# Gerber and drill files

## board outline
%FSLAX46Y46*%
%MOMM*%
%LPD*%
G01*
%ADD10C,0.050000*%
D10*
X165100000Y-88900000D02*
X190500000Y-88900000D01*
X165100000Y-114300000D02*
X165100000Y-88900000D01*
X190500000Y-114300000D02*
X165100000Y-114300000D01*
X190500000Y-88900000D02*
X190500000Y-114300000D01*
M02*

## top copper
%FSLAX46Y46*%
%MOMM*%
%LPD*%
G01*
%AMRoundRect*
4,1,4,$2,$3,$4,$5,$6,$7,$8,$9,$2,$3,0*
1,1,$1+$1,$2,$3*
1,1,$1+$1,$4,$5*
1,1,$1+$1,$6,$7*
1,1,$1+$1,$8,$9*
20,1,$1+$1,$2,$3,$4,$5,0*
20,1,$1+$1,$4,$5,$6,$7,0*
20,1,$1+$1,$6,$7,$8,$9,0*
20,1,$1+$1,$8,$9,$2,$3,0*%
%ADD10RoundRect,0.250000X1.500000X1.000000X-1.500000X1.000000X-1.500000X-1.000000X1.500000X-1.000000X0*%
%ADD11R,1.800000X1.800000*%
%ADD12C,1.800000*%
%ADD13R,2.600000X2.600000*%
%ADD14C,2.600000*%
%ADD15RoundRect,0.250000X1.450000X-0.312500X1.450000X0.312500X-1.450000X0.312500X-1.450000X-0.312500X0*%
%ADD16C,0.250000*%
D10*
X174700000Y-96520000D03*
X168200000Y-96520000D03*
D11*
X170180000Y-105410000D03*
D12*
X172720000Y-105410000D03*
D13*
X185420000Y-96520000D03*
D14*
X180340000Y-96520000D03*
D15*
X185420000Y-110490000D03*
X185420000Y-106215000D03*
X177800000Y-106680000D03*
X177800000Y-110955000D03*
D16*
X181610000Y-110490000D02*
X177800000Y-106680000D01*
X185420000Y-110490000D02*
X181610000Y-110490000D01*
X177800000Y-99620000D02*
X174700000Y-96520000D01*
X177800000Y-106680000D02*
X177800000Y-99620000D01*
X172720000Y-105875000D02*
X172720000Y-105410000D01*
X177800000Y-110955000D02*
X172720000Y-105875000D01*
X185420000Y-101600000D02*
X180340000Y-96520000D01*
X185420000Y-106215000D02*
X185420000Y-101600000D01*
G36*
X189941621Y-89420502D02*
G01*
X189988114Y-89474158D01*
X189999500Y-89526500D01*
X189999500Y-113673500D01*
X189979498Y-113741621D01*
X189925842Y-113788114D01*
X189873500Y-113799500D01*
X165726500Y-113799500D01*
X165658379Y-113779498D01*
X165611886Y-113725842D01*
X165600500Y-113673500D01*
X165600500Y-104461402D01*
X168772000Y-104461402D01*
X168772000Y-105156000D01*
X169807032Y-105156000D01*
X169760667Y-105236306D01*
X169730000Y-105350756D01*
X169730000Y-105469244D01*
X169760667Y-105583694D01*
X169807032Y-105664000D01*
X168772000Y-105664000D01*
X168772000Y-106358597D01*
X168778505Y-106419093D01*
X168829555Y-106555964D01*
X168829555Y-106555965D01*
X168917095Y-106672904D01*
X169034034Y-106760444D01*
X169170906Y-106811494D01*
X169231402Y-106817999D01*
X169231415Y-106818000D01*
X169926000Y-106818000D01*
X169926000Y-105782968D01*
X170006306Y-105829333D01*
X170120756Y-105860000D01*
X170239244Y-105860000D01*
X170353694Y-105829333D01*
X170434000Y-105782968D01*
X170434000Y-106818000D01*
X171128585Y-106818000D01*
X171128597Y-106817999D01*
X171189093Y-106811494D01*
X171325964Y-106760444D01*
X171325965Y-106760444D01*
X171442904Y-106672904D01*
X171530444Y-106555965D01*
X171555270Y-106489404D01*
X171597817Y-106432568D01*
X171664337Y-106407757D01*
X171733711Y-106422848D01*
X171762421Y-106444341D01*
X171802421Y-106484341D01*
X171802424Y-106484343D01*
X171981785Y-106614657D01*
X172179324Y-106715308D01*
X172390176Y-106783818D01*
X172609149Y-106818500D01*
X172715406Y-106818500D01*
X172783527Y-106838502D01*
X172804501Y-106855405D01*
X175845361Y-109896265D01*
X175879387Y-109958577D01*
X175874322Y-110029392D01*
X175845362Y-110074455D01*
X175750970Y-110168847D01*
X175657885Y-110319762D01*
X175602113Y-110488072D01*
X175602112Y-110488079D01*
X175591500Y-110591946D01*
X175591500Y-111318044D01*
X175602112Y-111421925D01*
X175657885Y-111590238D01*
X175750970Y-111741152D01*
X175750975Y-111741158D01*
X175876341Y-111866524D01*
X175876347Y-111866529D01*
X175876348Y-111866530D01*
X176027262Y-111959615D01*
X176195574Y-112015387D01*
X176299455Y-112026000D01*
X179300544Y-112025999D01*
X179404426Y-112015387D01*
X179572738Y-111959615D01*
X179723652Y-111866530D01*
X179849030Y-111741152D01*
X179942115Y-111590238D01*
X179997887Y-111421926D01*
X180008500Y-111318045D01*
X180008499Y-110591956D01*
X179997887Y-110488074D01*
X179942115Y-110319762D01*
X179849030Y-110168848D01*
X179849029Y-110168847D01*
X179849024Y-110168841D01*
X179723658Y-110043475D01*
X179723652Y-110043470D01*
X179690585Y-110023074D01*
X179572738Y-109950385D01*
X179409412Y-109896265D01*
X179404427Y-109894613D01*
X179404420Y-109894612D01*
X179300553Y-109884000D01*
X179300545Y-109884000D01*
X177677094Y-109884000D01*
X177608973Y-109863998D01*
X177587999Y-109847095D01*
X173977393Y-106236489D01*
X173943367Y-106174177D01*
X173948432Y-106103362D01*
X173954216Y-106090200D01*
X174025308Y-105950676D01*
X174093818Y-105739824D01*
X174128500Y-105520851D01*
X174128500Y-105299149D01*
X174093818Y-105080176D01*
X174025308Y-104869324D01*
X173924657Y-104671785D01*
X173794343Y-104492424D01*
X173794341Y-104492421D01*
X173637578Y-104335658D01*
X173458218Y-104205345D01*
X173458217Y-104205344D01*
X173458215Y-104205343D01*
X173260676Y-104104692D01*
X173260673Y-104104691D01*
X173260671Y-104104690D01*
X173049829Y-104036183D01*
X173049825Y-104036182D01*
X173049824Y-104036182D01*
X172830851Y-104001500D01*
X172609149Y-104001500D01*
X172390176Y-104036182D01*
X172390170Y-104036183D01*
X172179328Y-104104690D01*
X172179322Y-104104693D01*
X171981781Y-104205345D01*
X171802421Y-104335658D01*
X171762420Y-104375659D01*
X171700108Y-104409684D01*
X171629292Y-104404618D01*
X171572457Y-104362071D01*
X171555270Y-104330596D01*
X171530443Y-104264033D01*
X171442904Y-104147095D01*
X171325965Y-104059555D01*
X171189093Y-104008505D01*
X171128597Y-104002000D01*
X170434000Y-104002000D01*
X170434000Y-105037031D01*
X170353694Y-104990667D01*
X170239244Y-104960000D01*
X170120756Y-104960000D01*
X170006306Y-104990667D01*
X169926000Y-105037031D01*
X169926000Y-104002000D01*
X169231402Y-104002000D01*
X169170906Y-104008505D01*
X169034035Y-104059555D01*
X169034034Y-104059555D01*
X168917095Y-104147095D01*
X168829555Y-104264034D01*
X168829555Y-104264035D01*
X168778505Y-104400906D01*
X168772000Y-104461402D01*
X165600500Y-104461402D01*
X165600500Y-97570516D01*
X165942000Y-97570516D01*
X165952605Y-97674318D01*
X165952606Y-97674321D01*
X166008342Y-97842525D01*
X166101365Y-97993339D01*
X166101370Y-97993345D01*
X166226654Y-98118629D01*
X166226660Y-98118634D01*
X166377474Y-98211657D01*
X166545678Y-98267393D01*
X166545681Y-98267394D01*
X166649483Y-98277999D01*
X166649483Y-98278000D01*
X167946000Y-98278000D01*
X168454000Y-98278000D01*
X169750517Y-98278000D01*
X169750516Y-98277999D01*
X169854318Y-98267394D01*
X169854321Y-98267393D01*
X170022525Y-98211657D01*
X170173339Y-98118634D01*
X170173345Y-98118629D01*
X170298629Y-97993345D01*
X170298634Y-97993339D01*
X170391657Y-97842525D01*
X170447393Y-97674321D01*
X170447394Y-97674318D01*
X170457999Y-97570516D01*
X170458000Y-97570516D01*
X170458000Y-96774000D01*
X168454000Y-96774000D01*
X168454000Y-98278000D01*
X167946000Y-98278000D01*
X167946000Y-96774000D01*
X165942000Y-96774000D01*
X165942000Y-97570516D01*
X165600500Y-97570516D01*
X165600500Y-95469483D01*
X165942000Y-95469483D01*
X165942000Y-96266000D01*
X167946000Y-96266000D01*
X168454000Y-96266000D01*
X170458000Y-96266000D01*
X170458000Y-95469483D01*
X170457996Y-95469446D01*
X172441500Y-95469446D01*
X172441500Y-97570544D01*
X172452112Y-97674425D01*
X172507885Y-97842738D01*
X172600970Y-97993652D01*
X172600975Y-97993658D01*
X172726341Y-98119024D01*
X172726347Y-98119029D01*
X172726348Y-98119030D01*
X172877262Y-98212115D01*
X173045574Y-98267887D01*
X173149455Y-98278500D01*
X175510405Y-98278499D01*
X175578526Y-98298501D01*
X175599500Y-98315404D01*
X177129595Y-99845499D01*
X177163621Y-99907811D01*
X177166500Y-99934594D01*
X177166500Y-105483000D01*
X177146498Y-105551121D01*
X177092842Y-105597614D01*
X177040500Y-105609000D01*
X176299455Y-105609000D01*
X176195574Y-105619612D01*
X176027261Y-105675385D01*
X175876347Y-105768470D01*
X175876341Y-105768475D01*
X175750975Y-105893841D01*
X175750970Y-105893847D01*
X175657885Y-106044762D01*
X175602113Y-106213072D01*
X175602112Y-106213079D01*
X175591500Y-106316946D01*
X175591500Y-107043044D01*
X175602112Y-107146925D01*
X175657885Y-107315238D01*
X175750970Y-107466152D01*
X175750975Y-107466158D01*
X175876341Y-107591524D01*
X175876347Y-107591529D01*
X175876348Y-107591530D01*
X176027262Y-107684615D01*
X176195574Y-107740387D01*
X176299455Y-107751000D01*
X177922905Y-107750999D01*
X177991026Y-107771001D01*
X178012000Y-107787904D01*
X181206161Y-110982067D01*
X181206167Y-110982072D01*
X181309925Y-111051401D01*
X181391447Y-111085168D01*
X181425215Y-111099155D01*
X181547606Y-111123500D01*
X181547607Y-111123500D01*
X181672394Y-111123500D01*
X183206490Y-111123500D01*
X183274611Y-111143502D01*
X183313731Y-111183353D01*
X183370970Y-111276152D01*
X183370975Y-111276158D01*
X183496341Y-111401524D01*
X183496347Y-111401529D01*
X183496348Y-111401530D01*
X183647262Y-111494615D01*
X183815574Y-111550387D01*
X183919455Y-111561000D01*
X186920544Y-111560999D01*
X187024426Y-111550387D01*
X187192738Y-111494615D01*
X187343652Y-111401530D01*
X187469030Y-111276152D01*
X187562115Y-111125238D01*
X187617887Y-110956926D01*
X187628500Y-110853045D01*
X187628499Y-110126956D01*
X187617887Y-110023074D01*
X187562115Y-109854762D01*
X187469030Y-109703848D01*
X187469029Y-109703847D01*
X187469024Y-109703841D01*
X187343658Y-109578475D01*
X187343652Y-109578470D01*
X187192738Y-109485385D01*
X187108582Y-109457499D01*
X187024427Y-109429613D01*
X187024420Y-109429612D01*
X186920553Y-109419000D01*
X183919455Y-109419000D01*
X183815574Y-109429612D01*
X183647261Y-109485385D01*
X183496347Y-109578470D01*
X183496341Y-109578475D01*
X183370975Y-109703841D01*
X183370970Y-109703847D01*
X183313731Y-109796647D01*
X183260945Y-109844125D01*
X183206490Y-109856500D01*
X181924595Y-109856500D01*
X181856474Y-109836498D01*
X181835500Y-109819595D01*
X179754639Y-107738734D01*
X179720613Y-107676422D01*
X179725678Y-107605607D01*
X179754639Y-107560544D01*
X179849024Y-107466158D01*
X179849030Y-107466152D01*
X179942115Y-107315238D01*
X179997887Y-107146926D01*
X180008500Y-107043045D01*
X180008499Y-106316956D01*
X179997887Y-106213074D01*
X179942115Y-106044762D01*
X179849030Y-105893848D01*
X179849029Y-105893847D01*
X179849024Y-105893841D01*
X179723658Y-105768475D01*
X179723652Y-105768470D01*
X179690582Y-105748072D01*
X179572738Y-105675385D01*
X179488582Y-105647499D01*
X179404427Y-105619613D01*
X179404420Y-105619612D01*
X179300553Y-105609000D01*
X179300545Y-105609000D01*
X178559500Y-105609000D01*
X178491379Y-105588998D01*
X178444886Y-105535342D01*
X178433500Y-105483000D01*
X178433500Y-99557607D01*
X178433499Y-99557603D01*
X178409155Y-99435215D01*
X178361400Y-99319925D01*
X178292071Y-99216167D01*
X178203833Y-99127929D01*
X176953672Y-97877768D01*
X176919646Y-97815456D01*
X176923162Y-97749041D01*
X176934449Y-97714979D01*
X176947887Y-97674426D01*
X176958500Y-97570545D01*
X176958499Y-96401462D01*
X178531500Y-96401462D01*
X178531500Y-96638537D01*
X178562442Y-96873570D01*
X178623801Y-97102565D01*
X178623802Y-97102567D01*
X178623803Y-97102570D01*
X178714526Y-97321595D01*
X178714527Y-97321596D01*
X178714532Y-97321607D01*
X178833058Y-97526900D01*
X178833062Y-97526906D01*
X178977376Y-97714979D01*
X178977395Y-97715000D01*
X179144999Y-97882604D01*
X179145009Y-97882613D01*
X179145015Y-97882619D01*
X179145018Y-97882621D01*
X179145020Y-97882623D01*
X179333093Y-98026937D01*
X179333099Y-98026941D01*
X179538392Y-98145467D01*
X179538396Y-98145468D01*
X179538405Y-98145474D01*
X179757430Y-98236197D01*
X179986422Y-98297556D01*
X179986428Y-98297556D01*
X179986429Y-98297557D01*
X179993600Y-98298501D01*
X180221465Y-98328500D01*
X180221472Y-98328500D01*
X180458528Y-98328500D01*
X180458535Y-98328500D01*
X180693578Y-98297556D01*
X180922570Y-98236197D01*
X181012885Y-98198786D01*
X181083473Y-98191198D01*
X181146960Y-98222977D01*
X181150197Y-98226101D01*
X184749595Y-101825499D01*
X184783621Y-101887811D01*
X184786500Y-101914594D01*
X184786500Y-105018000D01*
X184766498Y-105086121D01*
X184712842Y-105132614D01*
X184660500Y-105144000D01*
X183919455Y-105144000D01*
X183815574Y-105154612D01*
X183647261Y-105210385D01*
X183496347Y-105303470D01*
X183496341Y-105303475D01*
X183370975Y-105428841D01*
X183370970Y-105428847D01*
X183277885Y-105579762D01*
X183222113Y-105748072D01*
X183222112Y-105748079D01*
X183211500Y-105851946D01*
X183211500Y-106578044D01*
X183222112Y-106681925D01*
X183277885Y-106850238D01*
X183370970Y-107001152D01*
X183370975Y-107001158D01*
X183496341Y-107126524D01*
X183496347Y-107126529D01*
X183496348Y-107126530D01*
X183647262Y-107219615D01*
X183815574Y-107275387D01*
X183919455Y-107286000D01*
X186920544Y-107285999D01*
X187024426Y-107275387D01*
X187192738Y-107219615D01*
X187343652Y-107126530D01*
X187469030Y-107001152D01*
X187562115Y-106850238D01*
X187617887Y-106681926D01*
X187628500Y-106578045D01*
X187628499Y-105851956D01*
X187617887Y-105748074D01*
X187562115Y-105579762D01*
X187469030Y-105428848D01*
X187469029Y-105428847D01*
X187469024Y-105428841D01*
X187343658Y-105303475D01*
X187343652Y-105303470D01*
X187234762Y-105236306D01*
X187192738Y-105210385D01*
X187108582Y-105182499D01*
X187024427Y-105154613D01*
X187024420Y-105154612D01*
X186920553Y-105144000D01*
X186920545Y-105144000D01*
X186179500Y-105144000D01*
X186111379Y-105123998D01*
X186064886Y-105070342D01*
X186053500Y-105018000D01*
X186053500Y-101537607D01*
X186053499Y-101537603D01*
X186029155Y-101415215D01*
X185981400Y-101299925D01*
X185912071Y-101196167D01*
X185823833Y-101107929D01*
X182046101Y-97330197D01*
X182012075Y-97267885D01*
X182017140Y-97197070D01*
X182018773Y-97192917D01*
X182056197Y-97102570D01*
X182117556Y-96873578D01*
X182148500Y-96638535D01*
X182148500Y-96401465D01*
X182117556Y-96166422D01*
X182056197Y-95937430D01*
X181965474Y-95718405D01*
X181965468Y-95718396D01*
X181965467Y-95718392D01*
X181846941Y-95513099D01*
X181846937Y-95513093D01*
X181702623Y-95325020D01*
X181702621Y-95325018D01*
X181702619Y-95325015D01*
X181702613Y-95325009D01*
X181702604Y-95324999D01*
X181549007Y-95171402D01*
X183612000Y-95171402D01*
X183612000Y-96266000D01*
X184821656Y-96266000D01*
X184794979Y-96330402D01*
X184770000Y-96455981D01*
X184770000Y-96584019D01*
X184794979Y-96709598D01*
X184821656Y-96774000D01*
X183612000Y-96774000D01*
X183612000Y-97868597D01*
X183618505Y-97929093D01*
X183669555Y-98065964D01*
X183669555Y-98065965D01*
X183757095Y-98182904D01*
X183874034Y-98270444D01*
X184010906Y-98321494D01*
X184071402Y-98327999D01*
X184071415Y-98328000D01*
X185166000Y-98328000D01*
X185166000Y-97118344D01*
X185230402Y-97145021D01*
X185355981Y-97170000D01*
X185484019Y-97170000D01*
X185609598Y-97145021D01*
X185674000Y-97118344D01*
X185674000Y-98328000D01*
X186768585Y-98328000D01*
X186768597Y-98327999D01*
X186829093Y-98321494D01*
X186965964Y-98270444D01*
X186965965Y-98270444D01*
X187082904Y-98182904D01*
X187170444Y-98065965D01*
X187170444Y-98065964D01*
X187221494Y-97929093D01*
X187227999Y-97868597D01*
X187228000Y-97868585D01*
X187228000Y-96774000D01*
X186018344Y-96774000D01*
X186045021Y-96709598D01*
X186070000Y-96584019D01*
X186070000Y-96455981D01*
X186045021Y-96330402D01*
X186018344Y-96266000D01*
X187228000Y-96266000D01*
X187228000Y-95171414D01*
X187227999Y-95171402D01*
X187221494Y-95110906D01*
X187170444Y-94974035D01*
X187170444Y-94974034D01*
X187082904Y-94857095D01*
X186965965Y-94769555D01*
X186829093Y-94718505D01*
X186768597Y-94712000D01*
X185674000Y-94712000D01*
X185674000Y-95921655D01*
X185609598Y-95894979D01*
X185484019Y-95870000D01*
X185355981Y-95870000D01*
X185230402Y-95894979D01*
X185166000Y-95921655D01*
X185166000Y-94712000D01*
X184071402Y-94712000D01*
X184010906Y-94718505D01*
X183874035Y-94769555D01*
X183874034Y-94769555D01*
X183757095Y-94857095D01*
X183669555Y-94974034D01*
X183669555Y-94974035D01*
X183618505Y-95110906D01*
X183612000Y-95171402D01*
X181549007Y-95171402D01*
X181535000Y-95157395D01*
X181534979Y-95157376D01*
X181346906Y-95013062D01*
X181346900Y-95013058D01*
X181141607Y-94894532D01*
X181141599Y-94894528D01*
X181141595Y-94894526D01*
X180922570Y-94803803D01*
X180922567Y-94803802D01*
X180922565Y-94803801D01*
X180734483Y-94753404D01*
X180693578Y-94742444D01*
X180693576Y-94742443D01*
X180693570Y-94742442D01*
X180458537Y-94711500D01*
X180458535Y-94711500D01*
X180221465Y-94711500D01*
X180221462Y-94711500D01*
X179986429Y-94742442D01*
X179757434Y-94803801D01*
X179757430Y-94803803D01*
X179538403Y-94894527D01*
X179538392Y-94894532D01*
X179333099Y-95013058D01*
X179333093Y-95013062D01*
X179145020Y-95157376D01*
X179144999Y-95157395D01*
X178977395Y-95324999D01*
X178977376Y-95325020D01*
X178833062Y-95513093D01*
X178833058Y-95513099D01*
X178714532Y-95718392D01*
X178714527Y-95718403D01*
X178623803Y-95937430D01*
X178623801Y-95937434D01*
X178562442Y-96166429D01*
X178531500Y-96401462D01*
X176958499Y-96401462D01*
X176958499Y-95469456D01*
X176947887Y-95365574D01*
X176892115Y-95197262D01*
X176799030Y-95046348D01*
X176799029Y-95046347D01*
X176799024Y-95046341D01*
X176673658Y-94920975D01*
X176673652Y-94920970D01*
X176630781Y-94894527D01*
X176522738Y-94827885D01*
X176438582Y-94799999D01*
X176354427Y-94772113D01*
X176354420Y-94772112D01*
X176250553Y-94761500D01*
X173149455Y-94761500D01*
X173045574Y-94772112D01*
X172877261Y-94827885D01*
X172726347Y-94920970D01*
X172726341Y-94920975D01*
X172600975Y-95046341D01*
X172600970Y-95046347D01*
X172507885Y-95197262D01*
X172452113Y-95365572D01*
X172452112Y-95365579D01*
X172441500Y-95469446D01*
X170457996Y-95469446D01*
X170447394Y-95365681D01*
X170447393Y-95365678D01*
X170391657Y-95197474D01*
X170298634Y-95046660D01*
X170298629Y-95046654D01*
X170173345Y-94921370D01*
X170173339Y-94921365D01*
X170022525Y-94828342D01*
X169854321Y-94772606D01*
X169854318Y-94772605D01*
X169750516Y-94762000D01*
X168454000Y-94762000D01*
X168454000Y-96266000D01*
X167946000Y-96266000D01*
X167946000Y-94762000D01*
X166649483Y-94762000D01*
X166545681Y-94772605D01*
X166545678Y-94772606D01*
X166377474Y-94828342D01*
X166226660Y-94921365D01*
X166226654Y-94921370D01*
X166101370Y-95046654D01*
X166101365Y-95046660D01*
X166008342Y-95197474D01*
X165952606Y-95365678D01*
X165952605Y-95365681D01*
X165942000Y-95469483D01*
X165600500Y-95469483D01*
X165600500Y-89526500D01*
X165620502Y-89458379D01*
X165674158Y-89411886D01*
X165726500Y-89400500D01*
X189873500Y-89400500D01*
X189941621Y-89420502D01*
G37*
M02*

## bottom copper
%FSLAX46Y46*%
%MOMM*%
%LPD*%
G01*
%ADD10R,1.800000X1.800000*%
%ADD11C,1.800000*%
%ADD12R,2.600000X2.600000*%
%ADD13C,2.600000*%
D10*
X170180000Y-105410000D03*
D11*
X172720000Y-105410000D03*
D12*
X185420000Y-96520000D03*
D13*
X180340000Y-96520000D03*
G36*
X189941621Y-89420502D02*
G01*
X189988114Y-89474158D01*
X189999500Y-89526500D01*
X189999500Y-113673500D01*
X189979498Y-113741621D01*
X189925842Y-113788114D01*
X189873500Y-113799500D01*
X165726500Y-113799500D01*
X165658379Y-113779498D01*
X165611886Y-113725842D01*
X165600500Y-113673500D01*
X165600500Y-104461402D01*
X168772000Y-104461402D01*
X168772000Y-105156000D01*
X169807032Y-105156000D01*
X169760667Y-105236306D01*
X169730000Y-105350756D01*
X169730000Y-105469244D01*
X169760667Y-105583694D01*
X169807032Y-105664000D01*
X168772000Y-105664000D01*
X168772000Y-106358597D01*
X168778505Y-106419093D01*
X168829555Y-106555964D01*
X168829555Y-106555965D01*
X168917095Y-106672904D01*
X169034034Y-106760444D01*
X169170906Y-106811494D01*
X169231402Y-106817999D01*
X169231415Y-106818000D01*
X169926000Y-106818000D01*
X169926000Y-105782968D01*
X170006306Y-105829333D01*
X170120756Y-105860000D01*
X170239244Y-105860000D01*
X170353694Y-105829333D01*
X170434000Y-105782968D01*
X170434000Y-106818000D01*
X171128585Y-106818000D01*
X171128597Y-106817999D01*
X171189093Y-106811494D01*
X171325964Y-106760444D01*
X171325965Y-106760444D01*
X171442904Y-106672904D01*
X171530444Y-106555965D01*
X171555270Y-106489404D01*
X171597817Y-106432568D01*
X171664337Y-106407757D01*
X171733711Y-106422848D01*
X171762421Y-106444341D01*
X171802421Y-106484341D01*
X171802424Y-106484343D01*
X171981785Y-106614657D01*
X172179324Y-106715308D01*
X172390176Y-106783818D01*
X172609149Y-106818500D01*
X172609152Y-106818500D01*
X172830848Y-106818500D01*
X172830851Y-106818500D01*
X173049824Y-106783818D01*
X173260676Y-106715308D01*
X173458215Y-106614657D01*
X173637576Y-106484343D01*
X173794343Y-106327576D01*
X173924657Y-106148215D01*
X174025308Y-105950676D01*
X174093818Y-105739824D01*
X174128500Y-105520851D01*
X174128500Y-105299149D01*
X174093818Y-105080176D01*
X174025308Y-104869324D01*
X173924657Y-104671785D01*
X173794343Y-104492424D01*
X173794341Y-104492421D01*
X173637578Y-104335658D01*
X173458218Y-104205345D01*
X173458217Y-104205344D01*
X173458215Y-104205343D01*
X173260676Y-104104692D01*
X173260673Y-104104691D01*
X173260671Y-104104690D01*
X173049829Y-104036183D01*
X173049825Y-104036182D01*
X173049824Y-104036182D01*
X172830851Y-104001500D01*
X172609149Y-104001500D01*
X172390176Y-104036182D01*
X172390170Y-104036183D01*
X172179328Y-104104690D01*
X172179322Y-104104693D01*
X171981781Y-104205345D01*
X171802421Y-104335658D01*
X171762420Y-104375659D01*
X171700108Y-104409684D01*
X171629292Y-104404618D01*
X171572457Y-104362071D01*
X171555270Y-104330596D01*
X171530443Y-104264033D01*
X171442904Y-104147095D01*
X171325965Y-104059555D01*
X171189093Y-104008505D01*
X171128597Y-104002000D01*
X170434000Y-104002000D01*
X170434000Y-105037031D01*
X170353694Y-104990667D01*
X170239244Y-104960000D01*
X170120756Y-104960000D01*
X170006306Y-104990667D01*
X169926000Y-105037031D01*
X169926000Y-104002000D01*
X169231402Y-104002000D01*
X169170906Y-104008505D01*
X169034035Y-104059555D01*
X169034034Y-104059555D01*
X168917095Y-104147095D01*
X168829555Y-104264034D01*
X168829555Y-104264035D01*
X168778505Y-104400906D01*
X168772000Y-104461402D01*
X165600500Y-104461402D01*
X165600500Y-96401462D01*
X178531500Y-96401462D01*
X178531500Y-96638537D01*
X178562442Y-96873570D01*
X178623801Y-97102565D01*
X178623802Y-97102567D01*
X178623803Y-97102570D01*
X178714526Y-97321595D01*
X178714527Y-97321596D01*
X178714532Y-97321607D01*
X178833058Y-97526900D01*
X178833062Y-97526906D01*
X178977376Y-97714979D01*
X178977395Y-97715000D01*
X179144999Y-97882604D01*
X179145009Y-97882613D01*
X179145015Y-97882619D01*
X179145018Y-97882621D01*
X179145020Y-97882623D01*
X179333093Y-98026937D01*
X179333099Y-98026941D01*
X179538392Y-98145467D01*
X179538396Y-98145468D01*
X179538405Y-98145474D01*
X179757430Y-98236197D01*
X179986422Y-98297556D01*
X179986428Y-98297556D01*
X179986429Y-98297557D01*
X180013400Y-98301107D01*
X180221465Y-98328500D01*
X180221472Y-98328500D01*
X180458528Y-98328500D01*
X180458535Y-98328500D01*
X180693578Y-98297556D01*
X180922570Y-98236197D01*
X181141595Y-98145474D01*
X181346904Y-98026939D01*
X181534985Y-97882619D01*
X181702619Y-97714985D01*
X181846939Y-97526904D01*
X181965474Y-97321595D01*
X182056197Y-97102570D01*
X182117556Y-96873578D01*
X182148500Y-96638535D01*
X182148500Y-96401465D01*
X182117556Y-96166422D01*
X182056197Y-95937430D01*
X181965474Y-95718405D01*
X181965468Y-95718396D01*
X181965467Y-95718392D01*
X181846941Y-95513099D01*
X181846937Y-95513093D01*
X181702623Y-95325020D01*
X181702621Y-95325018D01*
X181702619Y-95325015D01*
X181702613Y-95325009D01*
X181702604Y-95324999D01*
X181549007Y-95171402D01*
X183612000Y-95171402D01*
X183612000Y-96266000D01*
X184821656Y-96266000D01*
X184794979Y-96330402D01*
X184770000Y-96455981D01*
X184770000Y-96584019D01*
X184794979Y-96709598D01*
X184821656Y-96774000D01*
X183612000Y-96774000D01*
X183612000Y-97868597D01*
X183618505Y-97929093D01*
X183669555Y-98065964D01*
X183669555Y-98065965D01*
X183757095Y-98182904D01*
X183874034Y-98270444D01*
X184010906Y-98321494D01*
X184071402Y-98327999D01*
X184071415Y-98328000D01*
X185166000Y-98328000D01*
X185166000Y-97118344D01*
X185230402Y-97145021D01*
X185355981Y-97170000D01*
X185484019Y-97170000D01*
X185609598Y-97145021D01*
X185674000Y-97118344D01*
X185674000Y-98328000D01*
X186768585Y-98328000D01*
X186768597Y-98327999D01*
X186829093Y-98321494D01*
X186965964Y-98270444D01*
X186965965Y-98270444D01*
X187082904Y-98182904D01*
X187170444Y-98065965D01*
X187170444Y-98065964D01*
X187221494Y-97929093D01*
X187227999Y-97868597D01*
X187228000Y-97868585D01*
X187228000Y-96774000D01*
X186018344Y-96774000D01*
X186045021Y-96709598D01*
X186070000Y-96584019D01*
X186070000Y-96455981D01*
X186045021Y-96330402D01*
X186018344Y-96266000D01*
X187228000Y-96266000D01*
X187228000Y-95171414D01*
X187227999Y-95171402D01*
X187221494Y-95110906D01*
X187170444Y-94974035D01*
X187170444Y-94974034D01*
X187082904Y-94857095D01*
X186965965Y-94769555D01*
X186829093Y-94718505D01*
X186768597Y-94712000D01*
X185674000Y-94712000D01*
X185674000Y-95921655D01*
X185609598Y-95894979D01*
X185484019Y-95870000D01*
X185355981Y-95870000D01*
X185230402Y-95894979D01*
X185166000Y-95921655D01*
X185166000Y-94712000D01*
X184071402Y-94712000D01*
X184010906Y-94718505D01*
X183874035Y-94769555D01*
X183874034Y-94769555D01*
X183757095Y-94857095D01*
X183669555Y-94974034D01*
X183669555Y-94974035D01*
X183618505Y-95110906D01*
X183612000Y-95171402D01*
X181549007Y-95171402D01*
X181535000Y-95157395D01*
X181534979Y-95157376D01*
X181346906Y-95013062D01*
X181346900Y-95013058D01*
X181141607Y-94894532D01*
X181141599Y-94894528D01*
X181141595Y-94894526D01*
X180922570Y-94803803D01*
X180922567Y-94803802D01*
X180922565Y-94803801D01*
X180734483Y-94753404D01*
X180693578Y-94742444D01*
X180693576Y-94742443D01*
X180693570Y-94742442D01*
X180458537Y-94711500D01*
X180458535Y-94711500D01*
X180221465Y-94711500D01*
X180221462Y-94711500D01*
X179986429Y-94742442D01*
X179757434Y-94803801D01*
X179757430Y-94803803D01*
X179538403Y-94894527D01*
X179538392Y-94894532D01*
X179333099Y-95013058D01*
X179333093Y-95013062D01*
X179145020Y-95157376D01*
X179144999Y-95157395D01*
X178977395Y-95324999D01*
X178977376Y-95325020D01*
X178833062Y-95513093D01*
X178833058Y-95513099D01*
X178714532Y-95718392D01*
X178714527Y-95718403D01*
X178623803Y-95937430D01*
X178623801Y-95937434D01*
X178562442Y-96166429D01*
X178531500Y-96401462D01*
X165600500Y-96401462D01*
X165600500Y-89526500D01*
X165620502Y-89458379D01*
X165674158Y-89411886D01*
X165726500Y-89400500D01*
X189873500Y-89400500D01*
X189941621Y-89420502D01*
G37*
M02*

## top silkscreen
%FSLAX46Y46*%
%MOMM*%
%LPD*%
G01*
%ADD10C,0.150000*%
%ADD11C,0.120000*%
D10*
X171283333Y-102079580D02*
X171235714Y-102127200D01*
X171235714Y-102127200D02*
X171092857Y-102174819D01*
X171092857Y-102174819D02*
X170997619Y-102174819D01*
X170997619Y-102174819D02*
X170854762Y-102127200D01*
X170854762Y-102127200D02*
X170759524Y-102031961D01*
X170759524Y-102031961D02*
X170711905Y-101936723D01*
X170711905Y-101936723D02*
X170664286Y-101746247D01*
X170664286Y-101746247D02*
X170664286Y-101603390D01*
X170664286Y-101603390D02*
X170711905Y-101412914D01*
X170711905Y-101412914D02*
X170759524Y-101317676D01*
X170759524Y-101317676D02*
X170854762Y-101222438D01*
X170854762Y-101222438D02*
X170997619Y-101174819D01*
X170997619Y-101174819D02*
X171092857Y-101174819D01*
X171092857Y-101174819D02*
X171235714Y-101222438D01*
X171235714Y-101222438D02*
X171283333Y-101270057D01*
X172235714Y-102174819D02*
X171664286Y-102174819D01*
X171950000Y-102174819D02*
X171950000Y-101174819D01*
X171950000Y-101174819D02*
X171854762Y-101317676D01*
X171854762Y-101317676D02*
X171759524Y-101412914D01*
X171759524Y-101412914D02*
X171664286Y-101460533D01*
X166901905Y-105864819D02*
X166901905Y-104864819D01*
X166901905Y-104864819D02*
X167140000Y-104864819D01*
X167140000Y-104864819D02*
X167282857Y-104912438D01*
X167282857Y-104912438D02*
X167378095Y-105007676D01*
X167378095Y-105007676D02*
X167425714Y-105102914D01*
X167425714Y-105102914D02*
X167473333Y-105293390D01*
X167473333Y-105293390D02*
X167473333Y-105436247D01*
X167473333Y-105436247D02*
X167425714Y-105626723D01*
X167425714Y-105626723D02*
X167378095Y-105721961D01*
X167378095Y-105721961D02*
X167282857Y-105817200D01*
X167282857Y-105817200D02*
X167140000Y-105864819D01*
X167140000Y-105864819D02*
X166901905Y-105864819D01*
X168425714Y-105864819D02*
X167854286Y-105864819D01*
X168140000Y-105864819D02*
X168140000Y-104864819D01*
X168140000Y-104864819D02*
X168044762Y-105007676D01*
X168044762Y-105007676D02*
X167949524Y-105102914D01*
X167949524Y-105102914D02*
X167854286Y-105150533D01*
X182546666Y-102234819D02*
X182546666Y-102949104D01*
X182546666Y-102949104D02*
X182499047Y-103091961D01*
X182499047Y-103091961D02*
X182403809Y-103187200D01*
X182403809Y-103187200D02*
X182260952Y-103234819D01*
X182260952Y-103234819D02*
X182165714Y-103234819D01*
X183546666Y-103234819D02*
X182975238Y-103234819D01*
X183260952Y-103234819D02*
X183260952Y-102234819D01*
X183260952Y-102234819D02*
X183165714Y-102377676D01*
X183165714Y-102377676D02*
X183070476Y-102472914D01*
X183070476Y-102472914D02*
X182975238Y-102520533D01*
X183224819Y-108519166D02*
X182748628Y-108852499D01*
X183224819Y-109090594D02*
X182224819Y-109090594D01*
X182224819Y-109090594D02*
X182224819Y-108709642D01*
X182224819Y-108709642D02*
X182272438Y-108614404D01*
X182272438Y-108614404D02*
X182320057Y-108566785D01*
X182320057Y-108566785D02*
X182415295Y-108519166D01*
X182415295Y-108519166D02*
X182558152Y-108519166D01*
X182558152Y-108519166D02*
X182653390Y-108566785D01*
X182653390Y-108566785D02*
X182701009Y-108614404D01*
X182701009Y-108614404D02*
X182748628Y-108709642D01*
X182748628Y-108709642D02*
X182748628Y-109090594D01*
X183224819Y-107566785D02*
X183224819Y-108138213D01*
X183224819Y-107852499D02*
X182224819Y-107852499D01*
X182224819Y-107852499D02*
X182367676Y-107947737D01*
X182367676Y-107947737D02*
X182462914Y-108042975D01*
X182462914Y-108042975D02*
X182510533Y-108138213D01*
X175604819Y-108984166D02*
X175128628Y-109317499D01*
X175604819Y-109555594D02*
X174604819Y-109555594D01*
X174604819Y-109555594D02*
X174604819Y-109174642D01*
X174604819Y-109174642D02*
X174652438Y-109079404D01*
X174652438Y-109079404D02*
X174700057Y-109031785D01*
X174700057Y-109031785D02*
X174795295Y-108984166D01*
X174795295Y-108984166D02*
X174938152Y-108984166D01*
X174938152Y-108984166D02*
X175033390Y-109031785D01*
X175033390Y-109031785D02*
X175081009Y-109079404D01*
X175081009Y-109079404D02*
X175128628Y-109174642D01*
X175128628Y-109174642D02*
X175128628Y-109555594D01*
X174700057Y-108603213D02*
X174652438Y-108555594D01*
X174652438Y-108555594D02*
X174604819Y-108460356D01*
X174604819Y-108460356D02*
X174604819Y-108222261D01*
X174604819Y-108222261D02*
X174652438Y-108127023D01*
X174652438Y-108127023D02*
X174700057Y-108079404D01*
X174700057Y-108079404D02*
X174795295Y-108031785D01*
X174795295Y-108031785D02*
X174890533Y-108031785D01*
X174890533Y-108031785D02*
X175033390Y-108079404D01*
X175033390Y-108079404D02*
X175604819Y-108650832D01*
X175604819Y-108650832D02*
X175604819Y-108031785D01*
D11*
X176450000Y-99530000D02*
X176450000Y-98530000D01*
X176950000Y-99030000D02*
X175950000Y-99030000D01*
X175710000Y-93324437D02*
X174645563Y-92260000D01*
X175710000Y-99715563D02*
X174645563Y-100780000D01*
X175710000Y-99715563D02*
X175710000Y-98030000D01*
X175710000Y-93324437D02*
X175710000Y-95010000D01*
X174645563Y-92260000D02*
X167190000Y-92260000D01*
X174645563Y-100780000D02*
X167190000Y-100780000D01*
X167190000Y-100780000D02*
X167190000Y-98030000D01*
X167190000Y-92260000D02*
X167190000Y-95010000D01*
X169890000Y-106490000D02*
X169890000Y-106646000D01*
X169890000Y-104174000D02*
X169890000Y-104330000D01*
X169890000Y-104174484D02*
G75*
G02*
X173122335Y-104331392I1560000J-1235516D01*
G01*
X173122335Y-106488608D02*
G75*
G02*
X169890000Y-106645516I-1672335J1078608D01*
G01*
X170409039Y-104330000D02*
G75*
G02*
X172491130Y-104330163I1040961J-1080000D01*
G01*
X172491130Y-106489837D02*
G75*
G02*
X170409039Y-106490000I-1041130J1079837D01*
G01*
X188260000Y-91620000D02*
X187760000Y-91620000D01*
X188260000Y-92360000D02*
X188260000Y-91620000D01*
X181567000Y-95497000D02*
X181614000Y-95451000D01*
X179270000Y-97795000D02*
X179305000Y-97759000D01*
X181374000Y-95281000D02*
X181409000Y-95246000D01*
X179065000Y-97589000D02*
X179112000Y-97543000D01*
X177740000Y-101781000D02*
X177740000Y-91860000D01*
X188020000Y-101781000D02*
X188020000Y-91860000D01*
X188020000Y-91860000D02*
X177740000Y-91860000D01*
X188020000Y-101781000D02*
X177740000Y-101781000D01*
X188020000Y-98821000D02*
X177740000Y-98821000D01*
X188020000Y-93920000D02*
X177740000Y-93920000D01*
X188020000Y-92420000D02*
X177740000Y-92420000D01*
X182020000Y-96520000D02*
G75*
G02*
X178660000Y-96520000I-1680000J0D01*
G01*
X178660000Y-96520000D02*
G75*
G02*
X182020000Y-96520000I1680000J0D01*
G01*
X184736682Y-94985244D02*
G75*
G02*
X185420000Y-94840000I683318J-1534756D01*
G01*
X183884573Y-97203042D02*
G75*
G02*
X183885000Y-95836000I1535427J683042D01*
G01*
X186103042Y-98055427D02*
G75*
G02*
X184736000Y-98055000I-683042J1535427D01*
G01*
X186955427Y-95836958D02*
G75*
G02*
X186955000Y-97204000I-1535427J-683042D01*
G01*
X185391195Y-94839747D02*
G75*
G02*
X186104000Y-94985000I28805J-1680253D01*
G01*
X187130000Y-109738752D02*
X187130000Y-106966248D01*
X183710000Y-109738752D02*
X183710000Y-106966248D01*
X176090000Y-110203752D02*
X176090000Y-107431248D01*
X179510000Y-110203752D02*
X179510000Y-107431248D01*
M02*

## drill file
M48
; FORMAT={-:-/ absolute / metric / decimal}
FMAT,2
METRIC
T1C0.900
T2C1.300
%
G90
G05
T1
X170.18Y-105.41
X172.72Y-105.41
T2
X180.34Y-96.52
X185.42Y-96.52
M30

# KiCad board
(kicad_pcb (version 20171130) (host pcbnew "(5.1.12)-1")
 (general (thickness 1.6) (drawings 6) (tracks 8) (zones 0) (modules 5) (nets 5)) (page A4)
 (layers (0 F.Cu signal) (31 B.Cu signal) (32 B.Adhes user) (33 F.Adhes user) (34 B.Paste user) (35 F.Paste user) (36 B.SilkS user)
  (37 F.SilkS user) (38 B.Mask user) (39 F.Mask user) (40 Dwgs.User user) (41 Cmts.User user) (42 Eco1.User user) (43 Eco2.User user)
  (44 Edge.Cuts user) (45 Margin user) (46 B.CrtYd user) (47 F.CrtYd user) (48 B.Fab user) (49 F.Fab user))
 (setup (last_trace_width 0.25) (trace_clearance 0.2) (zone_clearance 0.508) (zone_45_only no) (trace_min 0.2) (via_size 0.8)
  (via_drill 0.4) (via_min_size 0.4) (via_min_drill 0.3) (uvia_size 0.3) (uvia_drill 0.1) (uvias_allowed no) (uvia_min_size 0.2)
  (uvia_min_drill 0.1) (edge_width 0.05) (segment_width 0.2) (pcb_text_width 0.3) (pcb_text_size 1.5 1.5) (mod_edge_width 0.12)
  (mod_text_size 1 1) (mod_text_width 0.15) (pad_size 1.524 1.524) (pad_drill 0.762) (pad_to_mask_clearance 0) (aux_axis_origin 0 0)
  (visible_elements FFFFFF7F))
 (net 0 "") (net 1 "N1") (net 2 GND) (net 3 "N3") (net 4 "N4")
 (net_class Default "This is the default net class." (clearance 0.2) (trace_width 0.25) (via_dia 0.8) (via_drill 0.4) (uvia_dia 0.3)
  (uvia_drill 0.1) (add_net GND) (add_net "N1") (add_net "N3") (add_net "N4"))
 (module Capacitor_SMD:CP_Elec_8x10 (layer F.Cu) (at 171.45 96.52 180)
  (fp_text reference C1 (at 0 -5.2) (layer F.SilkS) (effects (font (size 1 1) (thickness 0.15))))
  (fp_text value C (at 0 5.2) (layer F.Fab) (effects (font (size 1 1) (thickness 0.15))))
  (fp_line (start -5 -3.01) (end -5 -2.01) (layer F.SilkS) (width 0.12))
  (fp_line (start -5.5 -2.51) (end -4.5 -2.51) (layer F.SilkS) (width 0.12))
  (fp_line (start -4.26 3.195563) (end -3.195563 4.26) (layer F.SilkS) (width 0.12))
  (fp_line (start -4.26 -3.195563) (end -3.195563 -4.26) (layer F.SilkS) (width 0.12))
  (fp_line (start -4.26 -3.195563) (end -4.26 -1.51) (layer F.SilkS) (width 0.12))
  (fp_line (start -4.26 3.195563) (end -4.26 1.51) (layer F.SilkS) (width 0.12))
  (fp_line (start -3.195563 4.26) (end 4.26 4.26) (layer F.SilkS) (width 0.12))
  (fp_line (start -3.195563 -4.26) (end 4.26 -4.26) (layer F.SilkS) (width 0.12))
  (fp_line (start 4.26 -4.26) (end 4.26 -1.51) (layer F.SilkS) (width 0.12))
  (fp_line (start 4.26 4.26) (end 4.26 1.51) (layer F.SilkS) (width 0.12))
  (pad 1 smd roundrect (at -3.25 0 180) (size 3.5 2.5) (layers F.Cu F.Paste F.Mask) (roundrect_rratio 0.1) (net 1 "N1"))
  (pad 2 smd roundrect (at 3.25 0 180) (size 3.5 2.5) (layers F.Cu F.Paste F.Mask) (roundrect_rratio 0.1) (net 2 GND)))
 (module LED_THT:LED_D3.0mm (layer F.Cu) (at 170.18 105.41)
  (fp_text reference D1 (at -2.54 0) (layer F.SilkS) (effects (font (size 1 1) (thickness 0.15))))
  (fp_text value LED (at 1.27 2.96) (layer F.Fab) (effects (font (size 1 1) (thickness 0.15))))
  (fp_line (start -0.29 1.08) (end -0.29 1.236) (layer F.SilkS) (width 0.12))
  (fp_line (start -0.29 -1.236) (end -0.29 -1.08) (layer F.SilkS) (width 0.12))
  (fp_arc (start 1.27 0) (end -0.29 -1.235516) (angle 108.8) (layer F.SilkS) (width 0.12))
  (fp_arc (start 1.27 0) (end -0.29 1.235516) (angle -108.8) (layer F.SilkS) (width 0.12))
  (fp_arc (start 1.27 0) (end 0.229039 -1.08) (angle 87.9) (layer F.SilkS) (width 0.12))
  (fp_arc (start 1.27 0) (end 0.229039 1.08) (angle -87.9) (layer F.SilkS) (width 0.12))
  (pad 1 thru_hole rect (at 0 0) (size 1.8 1.8) (drill 0.9) (layers *.Cu *.Mask) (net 2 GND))
  (pad 2 thru_hole circle (at 2.54 0) (size 1.8 1.8) (drill 0.9) (layers *.Cu *.Mask) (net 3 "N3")))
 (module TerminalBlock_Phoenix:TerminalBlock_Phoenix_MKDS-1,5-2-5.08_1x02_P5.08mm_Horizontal (layer F.Cu) (at 185.42 96.52 180)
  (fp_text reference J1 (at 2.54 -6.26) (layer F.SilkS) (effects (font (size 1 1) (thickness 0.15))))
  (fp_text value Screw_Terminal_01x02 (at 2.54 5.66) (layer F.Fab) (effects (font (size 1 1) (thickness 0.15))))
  (fp_line (start -2.84 4.9) (end -2.34 4.9) (layer F.SilkS) (width 0.12))
  (fp_line (start -2.84 4.16) (end -2.84 4.9) (layer F.SilkS) (width 0.12))
  (fp_line (start 3.853 1.023) (end 3.806 1.069) (layer F.SilkS) (width 0.12))
  (fp_line (start 6.15 -1.275) (end 6.115 -1.239) (layer F.SilkS) (width 0.12))
  (fp_line (start 4.046 1.239) (end 4.011 1.274) (layer F.SilkS) (width 0.12))
  (fp_line (start 6.355 -1.069) (end 6.308 -1.023) (layer F.SilkS) (width 0.12))
  (fp_line (start 7.68 -5.261) (end 7.68 4.66) (layer F.SilkS) (width 0.12))
  (fp_line (start -2.6 -5.261) (end -2.6 4.66) (layer F.SilkS) (width 0.12))
  (fp_line (start -2.6 4.66) (end 7.68 4.66) (layer F.SilkS) (width 0.12))
  (fp_line (start -2.6 -5.261) (end 7.68 -5.261) (layer F.SilkS) (width 0.12))
  (fp_line (start -2.6 -2.301) (end 7.68 -2.301) (layer F.SilkS) (width 0.12))
  (fp_line (start -2.6 2.6) (end 7.68 2.6) (layer F.SilkS) (width 0.12))
  (fp_line (start -2.6 4.1) (end 7.68 4.1) (layer F.SilkS) (width 0.12))
  (fp_circle (center 5.08 0) (end 6.76 0) (layer F.SilkS) (width 0.12))
  (fp_arc (start 0 0) (end 0 1.68) (angle -24) (layer F.SilkS) (width 0.12))
  (fp_arc (start 0 0) (end 1.535 0.684) (angle -48) (layer F.SilkS) (width 0.12))
  (fp_arc (start 0 0) (end 0.684 -1.535) (angle -48) (layer F.SilkS) (width 0.12))
  (fp_arc (start 0 0) (end -1.535 -0.684) (angle -48) (layer F.SilkS) (width 0.12))
  (fp_arc (start 0 0) (end -0.684 1.535) (angle -25) (layer F.SilkS) (width 0.12))
  (pad 1 thru_hole rect (at 0 0 180) (size 2.6 2.6) (drill 1.3) (layers *.Cu *.Mask) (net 2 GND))
  (pad 2 thru_hole circle (at 5.08 0 180) (size 2.6 2.6) (drill 1.3) (layers *.Cu *.Mask) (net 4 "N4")))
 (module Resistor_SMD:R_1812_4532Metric (layer F.Cu) (at 185.42 108.3525 90)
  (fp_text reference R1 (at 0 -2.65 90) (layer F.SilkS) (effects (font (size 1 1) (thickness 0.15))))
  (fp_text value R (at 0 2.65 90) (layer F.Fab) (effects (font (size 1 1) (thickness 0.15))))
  (fp_line (start -1.386252 1.71) (end 1.386252 1.71) (layer F.SilkS) (width 0.12))
  (fp_line (start -1.386252 -1.71) (end 1.386252 -1.71) (layer F.SilkS) (width 0.12))
  (pad 1 smd roundrect (at -2.1375 0 90) (size 1.125 3.4) (layers F.Cu F.Paste F.Mask) (roundrect_rratio 0.222222) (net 1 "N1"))
  (pad 2 smd roundrect (at 2.1375 0 90) (size 1.125 3.4) (layers F.Cu F.Paste F.Mask) (roundrect_rratio 0.222222) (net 4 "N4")))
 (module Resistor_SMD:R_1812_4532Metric (layer F.Cu) (at 177.8 108.8175 90)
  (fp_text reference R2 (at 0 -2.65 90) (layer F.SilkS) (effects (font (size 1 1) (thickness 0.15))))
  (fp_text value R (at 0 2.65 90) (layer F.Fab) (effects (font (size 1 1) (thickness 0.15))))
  (fp_line (start -1.386252 -1.71) (end 1.386252 -1.71) (layer F.SilkS) (width 0.12))
  (fp_line (start -1.386252 1.71) (end 1.386252 1.71) (layer F.SilkS) (width 0.12))
  (pad 2 smd roundrect (at 2.1375 0 90) (size 1.125 3.4) (layers F.Cu F.Paste F.Mask) (roundrect_rratio 0.222222) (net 1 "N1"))
  (pad 1 smd roundrect (at -2.1375 0 90) (size 1.125 3.4) (layers F.Cu F.Paste F.Mask) (roundrect_rratio 0.222222) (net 3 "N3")))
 (gr_line (start 165.1 88.9) (end 190.5 88.9) (layer Edge.Cuts) (width 0.05))
 (gr_line (start 165.1 114.3) (end 165.1 88.9) (layer Edge.Cuts) (width 0.05))
 (gr_line (start 190.5 114.3) (end 165.1 114.3) (layer Edge.Cuts) (width 0.05))
 (gr_line (start 190.5 88.9) (end 190.5 114.3) (layer Edge.Cuts) (width 0.05))
 (segment (start 181.61 110.49) (end 177.8 106.68) (width 0.25) (layer F.Cu) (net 1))
 (segment (start 185.42 110.49) (end 181.61 110.49) (width 0.25) (layer F.Cu) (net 1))
 (segment (start 177.8 99.62) (end 174.7 96.52) (width 0.25) (layer F.Cu) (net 1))
 (segment (start 177.8 106.68) (end 177.8 99.62) (width 0.25) (layer F.Cu) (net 1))
 (segment (start 172.72 105.875) (end 172.72 105.41) (width 0.25) (layer F.Cu) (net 3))
 (segment (start 177.8 110.955) (end 172.72 105.875) (width 0.25) (layer F.Cu) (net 3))
 (segment (start 185.42 101.6) (end 180.34 96.52) (width 0.25) (layer F.Cu) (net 4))
 (segment (start 185.42 106.215) (end 185.42 101.6) (width 0.25) (layer F.Cu) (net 4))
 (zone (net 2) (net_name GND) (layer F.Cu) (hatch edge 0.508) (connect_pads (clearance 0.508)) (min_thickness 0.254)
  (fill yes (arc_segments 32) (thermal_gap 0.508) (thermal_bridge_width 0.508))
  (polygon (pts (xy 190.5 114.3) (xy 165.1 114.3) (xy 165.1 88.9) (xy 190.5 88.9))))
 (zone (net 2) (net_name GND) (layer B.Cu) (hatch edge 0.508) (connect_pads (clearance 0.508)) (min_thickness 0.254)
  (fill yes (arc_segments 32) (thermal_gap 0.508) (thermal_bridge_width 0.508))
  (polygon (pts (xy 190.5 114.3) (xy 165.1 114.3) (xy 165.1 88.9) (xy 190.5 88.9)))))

